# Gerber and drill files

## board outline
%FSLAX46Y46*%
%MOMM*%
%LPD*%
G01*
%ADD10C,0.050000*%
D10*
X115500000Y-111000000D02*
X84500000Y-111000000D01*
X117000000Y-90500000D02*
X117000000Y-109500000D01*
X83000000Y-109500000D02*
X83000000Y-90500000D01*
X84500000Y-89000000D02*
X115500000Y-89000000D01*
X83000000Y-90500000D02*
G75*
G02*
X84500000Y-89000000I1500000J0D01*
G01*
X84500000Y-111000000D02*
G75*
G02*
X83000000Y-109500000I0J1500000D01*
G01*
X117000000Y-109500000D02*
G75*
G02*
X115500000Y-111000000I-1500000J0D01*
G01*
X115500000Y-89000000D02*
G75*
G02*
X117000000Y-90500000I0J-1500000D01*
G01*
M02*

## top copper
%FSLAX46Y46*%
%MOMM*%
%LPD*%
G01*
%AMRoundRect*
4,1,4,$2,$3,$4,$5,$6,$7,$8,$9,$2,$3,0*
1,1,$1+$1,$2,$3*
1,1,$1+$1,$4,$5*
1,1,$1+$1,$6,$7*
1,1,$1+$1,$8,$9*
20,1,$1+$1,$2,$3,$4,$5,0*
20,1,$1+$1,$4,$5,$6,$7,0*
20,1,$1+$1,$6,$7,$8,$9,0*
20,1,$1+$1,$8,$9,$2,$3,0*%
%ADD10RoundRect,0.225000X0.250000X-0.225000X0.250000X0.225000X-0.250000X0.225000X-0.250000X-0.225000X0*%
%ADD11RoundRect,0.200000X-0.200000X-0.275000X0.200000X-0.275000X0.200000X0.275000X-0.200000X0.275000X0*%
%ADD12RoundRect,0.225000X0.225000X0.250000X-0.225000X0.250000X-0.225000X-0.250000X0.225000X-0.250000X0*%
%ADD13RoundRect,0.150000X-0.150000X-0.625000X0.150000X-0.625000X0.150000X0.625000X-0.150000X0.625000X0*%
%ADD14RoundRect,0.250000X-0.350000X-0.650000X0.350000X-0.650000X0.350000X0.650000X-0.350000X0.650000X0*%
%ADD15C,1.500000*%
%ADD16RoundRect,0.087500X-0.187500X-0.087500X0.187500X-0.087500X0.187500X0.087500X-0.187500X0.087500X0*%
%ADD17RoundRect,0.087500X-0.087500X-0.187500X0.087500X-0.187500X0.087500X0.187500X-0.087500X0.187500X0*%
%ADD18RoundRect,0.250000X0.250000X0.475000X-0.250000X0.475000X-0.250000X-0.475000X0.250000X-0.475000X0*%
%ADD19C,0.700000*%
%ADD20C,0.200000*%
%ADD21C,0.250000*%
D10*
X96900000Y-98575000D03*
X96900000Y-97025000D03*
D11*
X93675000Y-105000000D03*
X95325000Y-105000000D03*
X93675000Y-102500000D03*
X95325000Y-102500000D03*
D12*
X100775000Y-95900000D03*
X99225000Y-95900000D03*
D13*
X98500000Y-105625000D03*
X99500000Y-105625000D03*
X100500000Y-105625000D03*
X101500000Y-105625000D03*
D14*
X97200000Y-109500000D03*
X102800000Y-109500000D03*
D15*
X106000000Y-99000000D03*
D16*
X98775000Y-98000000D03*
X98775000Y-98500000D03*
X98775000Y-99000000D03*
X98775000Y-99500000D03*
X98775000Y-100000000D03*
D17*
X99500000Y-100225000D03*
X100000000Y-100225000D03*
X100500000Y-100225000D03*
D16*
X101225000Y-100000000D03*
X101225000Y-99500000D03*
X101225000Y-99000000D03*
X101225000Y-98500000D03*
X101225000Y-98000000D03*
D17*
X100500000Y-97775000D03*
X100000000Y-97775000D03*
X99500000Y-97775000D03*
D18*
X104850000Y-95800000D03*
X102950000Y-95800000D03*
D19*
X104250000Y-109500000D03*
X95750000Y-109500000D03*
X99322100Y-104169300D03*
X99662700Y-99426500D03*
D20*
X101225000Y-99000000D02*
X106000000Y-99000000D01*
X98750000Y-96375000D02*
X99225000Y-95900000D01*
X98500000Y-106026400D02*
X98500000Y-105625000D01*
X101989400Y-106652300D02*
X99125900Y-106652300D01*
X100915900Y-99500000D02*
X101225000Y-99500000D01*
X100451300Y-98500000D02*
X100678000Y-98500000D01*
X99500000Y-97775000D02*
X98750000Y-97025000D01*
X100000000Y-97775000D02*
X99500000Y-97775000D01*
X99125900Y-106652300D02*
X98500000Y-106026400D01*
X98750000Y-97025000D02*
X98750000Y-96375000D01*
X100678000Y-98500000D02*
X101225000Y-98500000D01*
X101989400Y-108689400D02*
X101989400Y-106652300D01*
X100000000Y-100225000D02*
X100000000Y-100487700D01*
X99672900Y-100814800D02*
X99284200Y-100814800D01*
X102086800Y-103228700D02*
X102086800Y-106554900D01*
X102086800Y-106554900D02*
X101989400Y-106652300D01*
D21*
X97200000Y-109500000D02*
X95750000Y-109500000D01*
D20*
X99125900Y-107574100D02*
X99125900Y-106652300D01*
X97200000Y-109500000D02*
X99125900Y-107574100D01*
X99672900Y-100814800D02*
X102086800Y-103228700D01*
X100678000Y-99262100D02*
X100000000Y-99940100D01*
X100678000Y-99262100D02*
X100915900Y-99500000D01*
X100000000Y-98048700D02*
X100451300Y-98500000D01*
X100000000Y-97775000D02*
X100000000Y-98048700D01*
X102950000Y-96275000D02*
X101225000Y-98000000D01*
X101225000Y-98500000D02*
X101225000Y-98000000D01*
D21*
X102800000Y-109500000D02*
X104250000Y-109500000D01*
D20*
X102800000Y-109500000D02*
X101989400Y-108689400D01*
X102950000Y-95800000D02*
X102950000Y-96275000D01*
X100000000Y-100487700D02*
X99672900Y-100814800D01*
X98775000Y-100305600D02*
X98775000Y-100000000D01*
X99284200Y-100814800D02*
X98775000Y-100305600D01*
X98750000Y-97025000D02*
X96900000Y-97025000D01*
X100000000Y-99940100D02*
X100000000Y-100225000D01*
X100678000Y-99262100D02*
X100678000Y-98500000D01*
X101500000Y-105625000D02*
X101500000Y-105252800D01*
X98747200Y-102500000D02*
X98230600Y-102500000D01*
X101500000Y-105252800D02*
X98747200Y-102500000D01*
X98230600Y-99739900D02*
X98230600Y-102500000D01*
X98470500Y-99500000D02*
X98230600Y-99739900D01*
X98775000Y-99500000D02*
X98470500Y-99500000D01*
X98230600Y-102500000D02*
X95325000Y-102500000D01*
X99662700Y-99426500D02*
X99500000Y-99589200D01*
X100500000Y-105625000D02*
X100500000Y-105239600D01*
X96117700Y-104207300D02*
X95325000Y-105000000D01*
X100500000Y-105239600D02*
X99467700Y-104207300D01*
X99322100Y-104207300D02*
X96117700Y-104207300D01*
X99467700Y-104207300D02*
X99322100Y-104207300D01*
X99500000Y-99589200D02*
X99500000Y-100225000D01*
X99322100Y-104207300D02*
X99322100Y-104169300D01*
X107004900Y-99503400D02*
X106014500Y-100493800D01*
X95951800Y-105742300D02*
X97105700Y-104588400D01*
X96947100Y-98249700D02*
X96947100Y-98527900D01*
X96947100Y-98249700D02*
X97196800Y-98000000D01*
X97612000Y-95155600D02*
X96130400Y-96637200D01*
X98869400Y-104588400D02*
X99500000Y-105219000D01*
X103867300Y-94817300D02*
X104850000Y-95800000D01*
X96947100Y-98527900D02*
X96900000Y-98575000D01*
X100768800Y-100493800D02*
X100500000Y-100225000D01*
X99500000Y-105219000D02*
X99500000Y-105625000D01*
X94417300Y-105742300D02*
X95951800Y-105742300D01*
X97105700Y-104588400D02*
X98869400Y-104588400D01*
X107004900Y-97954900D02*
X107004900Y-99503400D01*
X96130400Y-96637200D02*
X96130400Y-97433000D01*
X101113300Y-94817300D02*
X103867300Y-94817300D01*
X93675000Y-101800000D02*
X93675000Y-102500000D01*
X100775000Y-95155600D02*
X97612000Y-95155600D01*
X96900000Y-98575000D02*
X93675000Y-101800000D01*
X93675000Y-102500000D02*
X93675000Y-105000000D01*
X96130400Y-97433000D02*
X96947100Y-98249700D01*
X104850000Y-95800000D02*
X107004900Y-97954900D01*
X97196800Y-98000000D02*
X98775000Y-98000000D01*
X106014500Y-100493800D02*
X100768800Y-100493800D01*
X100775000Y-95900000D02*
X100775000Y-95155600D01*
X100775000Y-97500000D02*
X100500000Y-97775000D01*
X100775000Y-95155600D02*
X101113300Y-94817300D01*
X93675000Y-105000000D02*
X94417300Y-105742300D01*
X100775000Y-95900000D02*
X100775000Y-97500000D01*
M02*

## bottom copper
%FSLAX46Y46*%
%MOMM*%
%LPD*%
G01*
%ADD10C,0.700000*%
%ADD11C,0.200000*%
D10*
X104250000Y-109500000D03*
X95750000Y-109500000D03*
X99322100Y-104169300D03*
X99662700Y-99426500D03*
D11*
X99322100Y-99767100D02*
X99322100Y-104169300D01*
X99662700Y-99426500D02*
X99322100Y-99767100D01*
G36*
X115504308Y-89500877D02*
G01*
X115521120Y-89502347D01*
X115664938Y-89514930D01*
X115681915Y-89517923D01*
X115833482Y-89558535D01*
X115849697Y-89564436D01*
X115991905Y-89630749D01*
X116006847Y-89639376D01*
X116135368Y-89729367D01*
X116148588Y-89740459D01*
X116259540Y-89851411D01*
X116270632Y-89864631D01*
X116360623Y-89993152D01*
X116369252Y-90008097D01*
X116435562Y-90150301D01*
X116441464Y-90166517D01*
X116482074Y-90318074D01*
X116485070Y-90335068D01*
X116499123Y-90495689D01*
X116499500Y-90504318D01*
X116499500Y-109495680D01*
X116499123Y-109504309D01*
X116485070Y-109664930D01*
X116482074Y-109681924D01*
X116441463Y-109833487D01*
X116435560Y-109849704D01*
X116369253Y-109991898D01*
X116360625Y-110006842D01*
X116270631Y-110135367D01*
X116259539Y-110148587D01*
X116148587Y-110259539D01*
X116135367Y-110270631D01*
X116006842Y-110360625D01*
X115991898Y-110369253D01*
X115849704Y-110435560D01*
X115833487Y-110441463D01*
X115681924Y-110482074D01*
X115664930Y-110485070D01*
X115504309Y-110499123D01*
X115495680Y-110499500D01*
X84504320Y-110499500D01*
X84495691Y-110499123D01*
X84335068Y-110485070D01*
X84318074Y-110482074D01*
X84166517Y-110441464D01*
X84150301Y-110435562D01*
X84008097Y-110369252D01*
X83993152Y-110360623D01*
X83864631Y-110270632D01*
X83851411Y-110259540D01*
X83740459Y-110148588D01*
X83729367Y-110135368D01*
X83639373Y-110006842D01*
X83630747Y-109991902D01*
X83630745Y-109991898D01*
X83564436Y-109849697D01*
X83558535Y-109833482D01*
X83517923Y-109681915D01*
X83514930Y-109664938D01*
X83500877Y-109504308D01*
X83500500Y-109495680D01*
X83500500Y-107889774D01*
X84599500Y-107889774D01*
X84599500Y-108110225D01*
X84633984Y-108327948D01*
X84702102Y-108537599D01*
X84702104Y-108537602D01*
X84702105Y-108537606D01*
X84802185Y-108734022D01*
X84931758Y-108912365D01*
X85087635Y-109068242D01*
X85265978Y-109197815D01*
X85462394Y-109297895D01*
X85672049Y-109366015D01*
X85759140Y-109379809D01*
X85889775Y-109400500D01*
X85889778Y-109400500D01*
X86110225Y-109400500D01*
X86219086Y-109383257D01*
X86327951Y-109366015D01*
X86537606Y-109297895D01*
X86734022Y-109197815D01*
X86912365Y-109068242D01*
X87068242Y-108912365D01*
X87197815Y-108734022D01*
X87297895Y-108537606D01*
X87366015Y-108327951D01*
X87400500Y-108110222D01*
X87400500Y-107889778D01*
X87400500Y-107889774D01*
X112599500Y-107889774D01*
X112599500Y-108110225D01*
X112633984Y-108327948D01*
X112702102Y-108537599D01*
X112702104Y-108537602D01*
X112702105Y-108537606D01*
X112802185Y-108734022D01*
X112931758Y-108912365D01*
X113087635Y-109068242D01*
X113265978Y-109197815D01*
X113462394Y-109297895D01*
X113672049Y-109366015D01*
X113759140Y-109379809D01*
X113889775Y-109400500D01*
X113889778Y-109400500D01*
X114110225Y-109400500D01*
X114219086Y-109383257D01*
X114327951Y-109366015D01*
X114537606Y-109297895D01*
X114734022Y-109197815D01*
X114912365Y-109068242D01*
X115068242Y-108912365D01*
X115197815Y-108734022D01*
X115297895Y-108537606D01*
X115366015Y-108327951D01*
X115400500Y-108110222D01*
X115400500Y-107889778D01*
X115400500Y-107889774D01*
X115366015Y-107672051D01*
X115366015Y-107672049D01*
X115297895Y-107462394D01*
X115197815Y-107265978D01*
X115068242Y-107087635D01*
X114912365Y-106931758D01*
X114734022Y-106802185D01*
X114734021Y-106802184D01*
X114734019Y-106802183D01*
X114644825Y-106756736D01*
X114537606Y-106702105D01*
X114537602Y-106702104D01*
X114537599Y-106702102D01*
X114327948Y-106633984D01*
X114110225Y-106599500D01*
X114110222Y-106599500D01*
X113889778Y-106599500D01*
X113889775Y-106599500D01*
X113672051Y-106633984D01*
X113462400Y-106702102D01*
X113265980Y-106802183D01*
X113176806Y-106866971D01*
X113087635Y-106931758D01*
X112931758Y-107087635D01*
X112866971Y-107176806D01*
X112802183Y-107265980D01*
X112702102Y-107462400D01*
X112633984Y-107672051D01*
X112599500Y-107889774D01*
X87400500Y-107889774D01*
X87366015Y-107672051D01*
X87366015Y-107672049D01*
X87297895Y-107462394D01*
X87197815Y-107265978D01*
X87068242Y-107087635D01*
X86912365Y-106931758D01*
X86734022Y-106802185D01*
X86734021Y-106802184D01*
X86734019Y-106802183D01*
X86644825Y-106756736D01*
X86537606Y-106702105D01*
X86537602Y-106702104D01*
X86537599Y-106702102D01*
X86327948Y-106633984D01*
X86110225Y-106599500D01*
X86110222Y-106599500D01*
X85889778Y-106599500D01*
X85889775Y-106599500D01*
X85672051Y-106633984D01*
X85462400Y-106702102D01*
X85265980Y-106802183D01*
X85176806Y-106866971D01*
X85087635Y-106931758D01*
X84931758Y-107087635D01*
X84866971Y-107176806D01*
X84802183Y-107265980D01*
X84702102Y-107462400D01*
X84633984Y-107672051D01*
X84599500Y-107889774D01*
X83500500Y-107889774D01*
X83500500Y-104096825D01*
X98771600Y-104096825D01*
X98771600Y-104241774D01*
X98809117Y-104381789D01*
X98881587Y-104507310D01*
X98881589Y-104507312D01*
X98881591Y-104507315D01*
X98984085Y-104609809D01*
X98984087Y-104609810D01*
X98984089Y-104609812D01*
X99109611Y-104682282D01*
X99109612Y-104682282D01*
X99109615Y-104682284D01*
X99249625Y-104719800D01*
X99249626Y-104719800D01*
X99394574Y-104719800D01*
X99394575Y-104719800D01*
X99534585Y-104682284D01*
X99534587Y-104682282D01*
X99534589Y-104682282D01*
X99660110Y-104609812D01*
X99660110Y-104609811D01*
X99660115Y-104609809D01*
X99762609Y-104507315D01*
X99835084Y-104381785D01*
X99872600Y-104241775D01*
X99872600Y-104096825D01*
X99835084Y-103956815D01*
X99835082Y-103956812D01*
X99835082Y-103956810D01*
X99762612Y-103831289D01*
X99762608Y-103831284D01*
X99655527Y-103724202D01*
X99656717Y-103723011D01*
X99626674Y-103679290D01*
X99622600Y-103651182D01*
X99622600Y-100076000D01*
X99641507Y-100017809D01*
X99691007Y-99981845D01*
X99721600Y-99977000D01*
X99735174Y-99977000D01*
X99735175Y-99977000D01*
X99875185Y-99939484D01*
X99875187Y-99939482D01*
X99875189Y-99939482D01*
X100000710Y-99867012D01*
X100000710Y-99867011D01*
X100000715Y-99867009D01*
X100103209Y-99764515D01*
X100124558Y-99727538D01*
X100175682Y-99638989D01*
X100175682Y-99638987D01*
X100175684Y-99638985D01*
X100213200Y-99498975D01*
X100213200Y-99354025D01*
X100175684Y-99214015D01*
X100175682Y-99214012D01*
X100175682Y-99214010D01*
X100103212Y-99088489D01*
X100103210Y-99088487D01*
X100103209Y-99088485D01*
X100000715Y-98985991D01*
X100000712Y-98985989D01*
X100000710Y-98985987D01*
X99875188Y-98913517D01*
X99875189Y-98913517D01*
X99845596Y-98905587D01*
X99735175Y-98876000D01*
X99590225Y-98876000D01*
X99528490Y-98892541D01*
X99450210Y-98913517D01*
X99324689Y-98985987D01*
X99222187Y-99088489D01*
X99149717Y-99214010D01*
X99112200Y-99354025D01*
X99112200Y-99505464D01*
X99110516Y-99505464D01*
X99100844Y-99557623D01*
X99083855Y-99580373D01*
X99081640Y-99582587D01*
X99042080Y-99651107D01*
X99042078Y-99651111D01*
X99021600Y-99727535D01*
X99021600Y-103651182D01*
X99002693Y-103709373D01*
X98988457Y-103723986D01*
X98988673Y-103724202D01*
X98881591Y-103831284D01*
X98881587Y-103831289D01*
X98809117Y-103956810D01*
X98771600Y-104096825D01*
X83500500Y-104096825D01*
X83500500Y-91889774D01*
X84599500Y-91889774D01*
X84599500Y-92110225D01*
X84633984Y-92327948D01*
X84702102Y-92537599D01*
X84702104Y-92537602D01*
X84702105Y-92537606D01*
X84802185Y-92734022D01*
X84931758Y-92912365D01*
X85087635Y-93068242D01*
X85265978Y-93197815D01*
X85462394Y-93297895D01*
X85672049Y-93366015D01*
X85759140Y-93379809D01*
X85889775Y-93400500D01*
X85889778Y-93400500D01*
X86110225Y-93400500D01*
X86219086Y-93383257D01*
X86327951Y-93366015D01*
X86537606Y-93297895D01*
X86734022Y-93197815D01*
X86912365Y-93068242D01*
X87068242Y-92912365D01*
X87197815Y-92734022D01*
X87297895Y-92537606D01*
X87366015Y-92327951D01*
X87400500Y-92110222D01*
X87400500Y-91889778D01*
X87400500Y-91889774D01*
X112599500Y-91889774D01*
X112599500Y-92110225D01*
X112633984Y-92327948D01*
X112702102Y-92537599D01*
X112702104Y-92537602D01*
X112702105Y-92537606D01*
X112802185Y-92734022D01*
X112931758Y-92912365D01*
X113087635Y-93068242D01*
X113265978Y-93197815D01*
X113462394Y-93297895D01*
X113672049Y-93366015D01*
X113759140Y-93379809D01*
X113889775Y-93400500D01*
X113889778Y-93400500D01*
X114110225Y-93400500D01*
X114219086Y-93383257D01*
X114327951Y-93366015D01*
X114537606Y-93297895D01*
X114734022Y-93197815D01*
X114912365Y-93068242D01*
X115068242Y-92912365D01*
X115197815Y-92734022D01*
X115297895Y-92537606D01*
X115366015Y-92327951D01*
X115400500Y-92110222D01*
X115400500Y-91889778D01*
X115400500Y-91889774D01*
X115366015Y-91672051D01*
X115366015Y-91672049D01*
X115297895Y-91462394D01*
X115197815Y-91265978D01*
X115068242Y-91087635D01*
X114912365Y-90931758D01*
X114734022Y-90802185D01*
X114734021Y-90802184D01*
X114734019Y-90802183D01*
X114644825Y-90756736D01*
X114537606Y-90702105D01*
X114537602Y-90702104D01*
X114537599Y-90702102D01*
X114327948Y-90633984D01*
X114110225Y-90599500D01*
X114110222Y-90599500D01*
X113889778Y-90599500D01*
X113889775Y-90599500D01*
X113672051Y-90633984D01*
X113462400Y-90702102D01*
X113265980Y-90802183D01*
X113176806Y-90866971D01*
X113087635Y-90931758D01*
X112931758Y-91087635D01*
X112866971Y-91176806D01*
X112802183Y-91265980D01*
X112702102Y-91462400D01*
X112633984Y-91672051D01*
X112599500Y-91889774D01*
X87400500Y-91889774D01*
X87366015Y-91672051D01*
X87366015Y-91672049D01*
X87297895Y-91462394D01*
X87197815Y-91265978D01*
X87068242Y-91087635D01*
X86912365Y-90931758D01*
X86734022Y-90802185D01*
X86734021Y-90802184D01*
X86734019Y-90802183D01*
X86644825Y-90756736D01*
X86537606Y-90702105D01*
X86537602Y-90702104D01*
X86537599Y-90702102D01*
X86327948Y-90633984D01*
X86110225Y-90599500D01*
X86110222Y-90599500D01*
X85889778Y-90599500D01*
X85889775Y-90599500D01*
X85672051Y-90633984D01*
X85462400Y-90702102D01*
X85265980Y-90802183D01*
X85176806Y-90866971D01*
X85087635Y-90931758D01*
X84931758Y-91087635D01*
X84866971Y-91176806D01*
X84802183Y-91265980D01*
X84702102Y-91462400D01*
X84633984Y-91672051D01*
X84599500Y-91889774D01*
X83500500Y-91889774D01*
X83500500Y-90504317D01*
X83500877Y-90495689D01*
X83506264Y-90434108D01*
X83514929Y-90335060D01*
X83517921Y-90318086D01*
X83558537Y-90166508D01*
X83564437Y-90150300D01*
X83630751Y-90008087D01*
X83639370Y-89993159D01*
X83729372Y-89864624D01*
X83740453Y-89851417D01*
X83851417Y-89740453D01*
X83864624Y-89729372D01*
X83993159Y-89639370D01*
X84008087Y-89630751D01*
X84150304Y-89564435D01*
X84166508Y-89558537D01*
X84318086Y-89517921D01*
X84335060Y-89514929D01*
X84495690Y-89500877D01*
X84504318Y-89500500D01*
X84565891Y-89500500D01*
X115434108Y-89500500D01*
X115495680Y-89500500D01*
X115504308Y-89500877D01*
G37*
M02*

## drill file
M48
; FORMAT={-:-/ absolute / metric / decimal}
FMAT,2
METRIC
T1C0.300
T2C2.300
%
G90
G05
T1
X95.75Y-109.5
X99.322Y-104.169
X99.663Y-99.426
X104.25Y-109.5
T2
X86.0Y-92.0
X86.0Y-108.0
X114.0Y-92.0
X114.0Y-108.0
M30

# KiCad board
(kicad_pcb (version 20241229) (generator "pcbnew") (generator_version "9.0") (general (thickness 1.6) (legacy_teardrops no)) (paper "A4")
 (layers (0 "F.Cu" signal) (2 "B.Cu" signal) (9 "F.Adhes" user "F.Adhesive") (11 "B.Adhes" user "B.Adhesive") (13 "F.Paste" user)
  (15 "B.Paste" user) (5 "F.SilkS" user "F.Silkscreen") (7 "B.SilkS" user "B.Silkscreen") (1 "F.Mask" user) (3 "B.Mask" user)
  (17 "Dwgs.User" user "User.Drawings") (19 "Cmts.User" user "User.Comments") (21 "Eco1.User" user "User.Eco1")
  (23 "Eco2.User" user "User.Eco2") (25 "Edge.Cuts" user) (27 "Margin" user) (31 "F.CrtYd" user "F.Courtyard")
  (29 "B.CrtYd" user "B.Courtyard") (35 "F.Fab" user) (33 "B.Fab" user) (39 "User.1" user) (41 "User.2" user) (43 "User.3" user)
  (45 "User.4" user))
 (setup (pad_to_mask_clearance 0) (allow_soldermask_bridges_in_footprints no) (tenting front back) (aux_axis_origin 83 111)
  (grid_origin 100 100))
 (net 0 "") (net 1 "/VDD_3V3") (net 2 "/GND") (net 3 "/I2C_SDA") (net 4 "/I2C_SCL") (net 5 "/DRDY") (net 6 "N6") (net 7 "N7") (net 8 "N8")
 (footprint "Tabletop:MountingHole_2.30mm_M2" (layer "F.Cu") (at 86 108)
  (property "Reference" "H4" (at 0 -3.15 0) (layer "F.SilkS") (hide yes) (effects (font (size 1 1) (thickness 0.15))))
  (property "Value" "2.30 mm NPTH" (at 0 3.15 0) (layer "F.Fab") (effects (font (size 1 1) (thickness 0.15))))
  (pad "" np_thru_hole circle (at 0 0) (size 2.3 2.3) (drill 2.3) (layers "*.Cu" "*.Mask")))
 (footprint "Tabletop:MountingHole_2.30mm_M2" (layer "F.Cu") (at 114 92)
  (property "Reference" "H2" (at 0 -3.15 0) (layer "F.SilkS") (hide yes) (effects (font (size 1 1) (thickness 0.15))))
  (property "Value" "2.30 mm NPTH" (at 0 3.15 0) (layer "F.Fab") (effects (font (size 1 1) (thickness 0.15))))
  (pad "" np_thru_hole circle (at 0 0) (size 2.3 2.3) (drill 2.3) (layers "*.Cu" "*.Mask")))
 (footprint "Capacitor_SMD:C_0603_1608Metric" (layer "F.Cu") (at 96.9 97.8 90)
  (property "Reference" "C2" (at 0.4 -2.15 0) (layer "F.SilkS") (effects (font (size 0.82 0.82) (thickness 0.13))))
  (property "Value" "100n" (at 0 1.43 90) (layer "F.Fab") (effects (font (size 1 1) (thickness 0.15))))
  (pad "1" smd roundrect (at -0.775 0 90) (size 0.9 0.95) (layers "F.Cu" "F.Mask" "F.Paste") (roundrect_rratio 0.25) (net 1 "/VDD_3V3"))
  (pad "2" smd roundrect (at 0.775 0 90) (size 0.9 0.95) (layers "F.Cu" "F.Mask" "F.Paste") (roundrect_rratio 0.25) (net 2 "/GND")))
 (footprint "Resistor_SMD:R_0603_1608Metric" (layer "F.Cu") (at 94.5 105)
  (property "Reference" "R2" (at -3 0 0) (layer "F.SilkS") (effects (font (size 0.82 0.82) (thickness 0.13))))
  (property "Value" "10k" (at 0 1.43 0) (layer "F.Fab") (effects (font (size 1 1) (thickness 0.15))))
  (pad "1" smd roundrect (at -0.825 0) (size 0.8 0.95) (layers "F.Cu" "F.Mask" "F.Paste") (roundrect_rratio 0.25) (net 1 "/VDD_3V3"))
  (pad "2" smd roundrect (at 0.825 0) (size 0.8 0.95) (layers "F.Cu" "F.Mask" "F.Paste") (roundrect_rratio 0.25) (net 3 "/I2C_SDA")))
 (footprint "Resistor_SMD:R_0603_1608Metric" (layer "F.Cu") (at 94.5 102.5)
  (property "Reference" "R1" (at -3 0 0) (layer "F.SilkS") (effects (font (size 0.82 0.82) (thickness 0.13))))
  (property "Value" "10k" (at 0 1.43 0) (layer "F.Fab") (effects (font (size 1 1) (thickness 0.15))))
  (pad "1" smd roundrect (at -0.825 0) (size 0.8 0.95) (layers "F.Cu" "F.Mask" "F.Paste") (roundrect_rratio 0.25) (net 1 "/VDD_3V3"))
  (pad "2" smd roundrect (at 0.825 0) (size 0.8 0.95) (layers "F.Cu" "F.Mask" "F.Paste") (roundrect_rratio 0.25) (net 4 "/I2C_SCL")))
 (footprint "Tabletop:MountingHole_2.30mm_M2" (layer "F.Cu") (at 114 108)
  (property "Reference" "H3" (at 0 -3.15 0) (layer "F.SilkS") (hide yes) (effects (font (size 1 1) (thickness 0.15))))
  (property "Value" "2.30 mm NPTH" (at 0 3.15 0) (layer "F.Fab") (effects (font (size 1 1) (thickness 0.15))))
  (pad "" np_thru_hole circle (at 0 0) (size 2.3 2.3) (drill 2.3) (layers "*.Cu" "*.Mask")))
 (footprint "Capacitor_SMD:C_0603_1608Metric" (layer "F.Cu") (at 100 95.9 180)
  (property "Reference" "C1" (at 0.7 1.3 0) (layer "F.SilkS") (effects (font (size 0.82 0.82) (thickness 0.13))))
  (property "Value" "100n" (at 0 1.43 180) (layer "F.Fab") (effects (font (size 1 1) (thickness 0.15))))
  (pad "1" smd roundrect (at -0.775 0 180) (size 0.9 0.95) (layers "F.Cu" "F.Mask" "F.Paste") (roundrect_rratio 0.25) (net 1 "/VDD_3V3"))
  (pad "2" smd roundrect (at 0.775 0 180) (size 0.9 0.95) (layers "F.Cu" "F.Mask" "F.Paste") (roundrect_rratio 0.25) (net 2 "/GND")))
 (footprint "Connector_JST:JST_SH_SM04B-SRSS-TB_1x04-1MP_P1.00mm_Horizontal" (layer "F.Cu") (at 100 107.625)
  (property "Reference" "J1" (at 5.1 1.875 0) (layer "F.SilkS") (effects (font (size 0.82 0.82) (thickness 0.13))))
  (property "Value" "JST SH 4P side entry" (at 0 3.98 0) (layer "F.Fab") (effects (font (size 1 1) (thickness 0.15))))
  (pad "1" smd roundrect (at -1.5 -2) (size 0.6 1.55) (layers "F.Cu" "F.Mask" "F.Paste") (roundrect_rratio 0.25) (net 2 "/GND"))
  (pad "2" smd roundrect (at -0.5 -2) (size 0.6 1.55) (layers "F.Cu" "F.Mask" "F.Paste") (roundrect_rratio 0.25) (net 1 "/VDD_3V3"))
  (pad "3" smd roundrect (at 0.5 -2) (size 0.6 1.55) (layers "F.Cu" "F.Mask" "F.Paste") (roundrect_rratio 0.25) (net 3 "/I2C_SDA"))
  (pad "4" smd roundrect (at 1.5 -2) (size 0.6 1.55) (layers "F.Cu" "F.Mask" "F.Paste") (roundrect_rratio 0.25) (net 4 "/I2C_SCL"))
  (pad "MP" smd roundrect (at -2.8 1.875) (size 1.2 1.8) (layers "F.Cu" "F.Mask" "F.Paste") (roundrect_rratio 0.208333) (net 2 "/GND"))
  (pad "MP" smd roundrect (at 2.8 1.875) (size 1.2 1.8) (layers "F.Cu" "F.Mask" "F.Paste") (roundrect_rratio 0.208333) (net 2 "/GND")))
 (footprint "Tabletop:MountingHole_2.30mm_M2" (layer "F.Cu") (at 86 92)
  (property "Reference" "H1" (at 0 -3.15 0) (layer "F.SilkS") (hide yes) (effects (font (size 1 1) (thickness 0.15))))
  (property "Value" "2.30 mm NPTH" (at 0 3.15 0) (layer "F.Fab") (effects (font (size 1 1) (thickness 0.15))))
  (pad "" np_thru_hole circle (at 0 0) (size 2.3 2.3) (drill 2.3) (layers "*.Cu" "*.Mask")))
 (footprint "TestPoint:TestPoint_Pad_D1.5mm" (layer "F.Cu") (at 106 99)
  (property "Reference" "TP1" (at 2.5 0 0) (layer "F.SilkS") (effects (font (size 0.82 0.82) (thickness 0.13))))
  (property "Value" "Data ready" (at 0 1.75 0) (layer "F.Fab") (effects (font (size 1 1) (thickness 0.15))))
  (pad "1" smd circle (at 0 0) (size 1.5 1.5) (layers "F.Cu" "F.Mask") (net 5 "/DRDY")))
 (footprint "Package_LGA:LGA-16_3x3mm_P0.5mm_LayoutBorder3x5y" (layer "F.Cu") (at 100 99)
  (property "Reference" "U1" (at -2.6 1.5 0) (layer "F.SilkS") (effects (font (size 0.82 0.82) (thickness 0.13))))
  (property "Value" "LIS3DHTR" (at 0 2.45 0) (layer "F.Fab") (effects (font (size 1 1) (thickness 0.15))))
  (pad "1" smd roundrect (at -1.225 -1) (size 0.55 0.35) (layers "F.Cu" "F.Mask" "F.Paste") (roundrect_rratio 0.25) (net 1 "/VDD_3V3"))
  (pad "2" smd roundrect (at -1.225 -0.5) (size 0.55 0.35) (layers "F.Cu" "F.Mask" "F.Paste") (roundrect_rratio 0.25) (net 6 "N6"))
  (pad "3" smd roundrect (at -1.225 0) (size 0.55 0.35) (layers "F.Cu" "F.Mask" "F.Paste") (roundrect_rratio 0.25) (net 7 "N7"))
  (pad "4" smd roundrect (at -1.225 0.5) (size 0.55 0.35) (layers "F.Cu" "F.Mask" "F.Paste") (roundrect_rratio 0.25) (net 4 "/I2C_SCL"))
  (pad "5" smd roundrect (at -1.225 1) (size 0.55 0.35) (layers "F.Cu" "F.Mask" "F.Paste") (roundrect_rratio 0.25) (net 2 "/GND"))
  (pad "6" smd roundrect (at -0.5 1.225) (size 0.35 0.55) (layers "F.Cu" "F.Mask" "F.Paste") (roundrect_rratio 0.25) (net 3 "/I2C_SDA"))
  (pad "7" smd roundrect (at 0 1.225) (size 0.35 0.55) (layers "F.Cu" "F.Mask" "F.Paste") (roundrect_rratio 0.25) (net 2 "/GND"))
  (pad "8" smd roundrect (at 0.5 1.225) (size 0.35 0.55) (layers "F.Cu" "F.Mask" "F.Paste") (roundrect_rratio 0.25) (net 1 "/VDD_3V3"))
  (pad "9" smd roundrect (at 1.225 1) (size 0.55 0.35) (layers "F.Cu" "F.Mask" "F.Paste") (roundrect_rratio 0.25) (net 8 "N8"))
  (pad "10" smd roundrect (at 1.225 0.5) (size 0.55 0.35) (layers "F.Cu" "F.Mask" "F.Paste") (roundrect_rratio 0.25) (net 2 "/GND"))
  (pad "11" smd roundrect (at 1.225 0) (size 0.55 0.35) (layers "F.Cu" "F.Mask" "F.Paste") (roundrect_rratio 0.25) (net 5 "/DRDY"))
  (pad "12" smd roundrect (at 1.225 -0.5) (size 0.55 0.35) (layers "F.Cu" "F.Mask" "F.Paste") (roundrect_rratio 0.25) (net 2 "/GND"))
  (pad "13" smd roundrect (at 1.225 -1) (size 0.55 0.35) (layers "F.Cu" "F.Mask" "F.Paste") (roundrect_rratio 0.25) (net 2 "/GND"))
  (pad "14" smd roundrect (at 0.5 -1.225) (size 0.35 0.55) (layers "F.Cu" "F.Mask" "F.Paste") (roundrect_rratio 0.25) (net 1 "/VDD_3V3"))
  (pad "15" smd roundrect (at 0 -1.225) (size 0.35 0.55) (layers "F.Cu" "F.Mask" "F.Paste") (roundrect_rratio 0.25) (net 2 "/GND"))
  (pad "16" smd roundrect (at -0.5 -1.225) (size 0.35 0.55) (layers "F.Cu" "F.Mask" "F.Paste") (roundrect_rratio 0.25) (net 2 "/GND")))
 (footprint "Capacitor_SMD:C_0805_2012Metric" (layer "F.Cu") (at 103.9 95.8 180)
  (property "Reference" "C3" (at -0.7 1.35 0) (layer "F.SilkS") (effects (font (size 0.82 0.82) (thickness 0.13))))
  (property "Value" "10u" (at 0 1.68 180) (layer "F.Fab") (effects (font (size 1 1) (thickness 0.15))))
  (pad "1" smd roundrect (at -0.95 0 180) (size 1 1.45) (layers "F.Cu" "F.Mask" "F.Paste") (roundrect_rratio 0.25) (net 1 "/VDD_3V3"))
  (pad "2" smd roundrect (at 0.95 0 180) (size 1 1.45) (layers "F.Cu" "F.Mask" "F.Paste") (roundrect_rratio 0.25) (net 2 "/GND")))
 (gr_line (start 115.5 111) (end 84.5 111) (stroke (width 0.05) (type default)) (layer "Edge.Cuts"))
 (gr_line (start 117 90.5) (end 117 109.5) (stroke (width 0.05) (type default)) (layer "Edge.Cuts"))
 (gr_line (start 83 109.5) (end 83 90.5) (stroke (width 0.05) (type default)) (layer "Edge.Cuts"))
 (gr_line (start 84.5 89) (end 115.5 89) (stroke (width 0.05) (type default)) (layer "Edge.Cuts"))
 (gr_arc (start 83 90.5) (mid 83.439339 89.439339) (end 84.5 89) (stroke (width 0.05) (type default)) (layer "Edge.Cuts"))
 (gr_arc (start 84.5 111) (mid 83.439339 110.56066) (end 83 109.5) (stroke (width 0.05) (type default)) (layer "Edge.Cuts"))
 (gr_arc (start 117 109.5) (mid 116.56066 110.56066) (end 115.5 111) (stroke (width 0.05) (type default)) (layer "Edge.Cuts"))
 (gr_arc (start 115.5 89) (mid 116.56066 89.439339) (end 117 90.5) (stroke (width 0.05) (type default)) (layer "Edge.Cuts"))
 (segment (start 101.225 99) (end 106 99) (width 0.2) (layer "F.Cu") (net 5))
 (segment (start 98.75 96.375) (end 99.225 95.9) (width 0.2) (layer "F.Cu") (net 2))
 (segment (start 98.5 106.0264) (end 98.5 105.625) (width 0.2) (layer "F.Cu") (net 2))
 (segment (start 101.9894 106.6523) (end 99.1259 106.6523) (width 0.2) (layer "F.Cu") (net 2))
 (segment (start 100.9159 99.5) (end 101.225 99.5) (width 0.2) (layer "F.Cu") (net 2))
 (segment (start 100.4513 98.5) (end 100.678 98.5) (width 0.2) (layer "F.Cu") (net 2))
 (segment (start 99.5 97.775) (end 98.75 97.025) (width 0.2) (layer "F.Cu") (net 2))
 (segment (start 100 97.775) (end 99.5 97.775) (width 0.2) (layer "F.Cu") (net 2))
 (segment (start 99.1259 106.6523) (end 98.5 106.0264) (width 0.2) (layer "F.Cu") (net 2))
 (segment (start 98.75 97.025) (end 98.75 96.375) (width 0.2) (layer "F.Cu") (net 2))
 (segment (start 100.678 98.5) (end 101.225 98.5) (width 0.2) (layer "F.Cu") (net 2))
 (segment (start 101.9894 108.6894) (end 101.9894 106.6523) (width 0.2) (layer "F.Cu") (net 2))
 (segment (start 100 100.225) (end 100 100.4877) (width 0.2) (layer "F.Cu") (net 2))
 (segment (start 99.6729 100.8148) (end 99.2842 100.8148) (width 0.2) (layer "F.Cu") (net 2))
 (segment (start 102.0868 103.2287) (end 102.0868 106.5549) (width 0.2) (layer "F.Cu") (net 2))
 (segment (start 102.0868 106.5549) (end 101.9894 106.6523) (width 0.2) (layer "F.Cu") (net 2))
 (segment (start 97.2 109.5) (end 95.75 109.5) (width 0.25) (layer "F.Cu") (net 2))
 (segment (start 99.1259 107.5741) (end 99.1259 106.6523) (width 0.2) (layer "F.Cu") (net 2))
 (segment (start 97.2 109.5) (end 99.1259 107.5741) (width 0.2) (layer "F.Cu") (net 2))
 (segment (start 99.6729 100.8148) (end 102.0868 103.2287) (width 0.2) (layer "F.Cu") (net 2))
 (segment (start 100.678 99.2621) (end 100 99.9401) (width 0.2) (layer "F.Cu") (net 2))
 (segment (start 100.678 99.2621) (end 100.9159 99.5) (width 0.2) (layer "F.Cu") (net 2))
 (segment (start 100 98.0487) (end 100.4513 98.5) (width 0.2) (layer "F.Cu") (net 2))
 (segment (start 100 97.775) (end 100 98.0487) (width 0.2) (layer "F.Cu") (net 2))
 (segment (start 102.95 96.275) (end 101.225 98) (width 0.2) (layer "F.Cu") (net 2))
 (segment (start 101.225 98.5) (end 101.225 98) (width 0.2) (layer "F.Cu") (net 2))
 (segment (start 102.8 109.5) (end 104.25 109.5) (width 0.25) (layer "F.Cu") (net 2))
 (segment (start 102.8 109.5) (end 101.9894 108.6894) (width 0.2) (layer "F.Cu") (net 2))
 (segment (start 102.95 95.8) (end 102.95 96.275) (width 0.2) (layer "F.Cu") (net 2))
 (segment (start 100 100.4877) (end 99.6729 100.8148) (width 0.2) (layer "F.Cu") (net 2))
 (segment (start 98.775 100.3056) (end 98.775 100) (width 0.2) (layer "F.Cu") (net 2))
 (segment (start 99.2842 100.8148) (end 98.775 100.3056) (width 0.2) (layer "F.Cu") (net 2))
 (segment (start 98.75 97.025) (end 96.9 97.025) (width 0.2) (layer "F.Cu") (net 2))
 (segment (start 100 99.9401) (end 100 100.225) (width 0.2) (layer "F.Cu") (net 2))
 (segment (start 100.678 99.2621) (end 100.678 98.5) (width 0.2) (layer "F.Cu") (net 2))
 (via (at 104.25 109.5) (size 0.7) (drill 0.3) (layers "F.Cu" "B.Cu") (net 2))
 (via (at 95.75 109.5) (size 0.7) (drill 0.3) (layers "F.Cu" "B.Cu") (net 2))
 (segment (start 101.5 105.625) (end 101.5 105.2528) (width 0.2) (layer "F.Cu") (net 4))
 (segment (start 98.7472 102.5) (end 98.2306 102.5) (width 0.2) (layer "F.Cu") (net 4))
 (segment (start 101.5 105.2528) (end 98.7472 102.5) (width 0.2) (layer "F.Cu") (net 4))
 (segment (start 98.2306 99.7399) (end 98.2306 102.5) (width 0.2) (layer "F.Cu") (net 4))
 (segment (start 98.4705 99.5) (end 98.2306 99.7399) (width 0.2) (layer "F.Cu") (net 4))
 (segment (start 98.775 99.5) (end 98.4705 99.5) (width 0.2) (layer "F.Cu") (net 4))
 (segment (start 98.2306 102.5) (end 95.325 102.5) (width 0.2) (layer "F.Cu") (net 4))
 (segment (start 99.6627 99.4265) (end 99.5 99.5892) (width 0.2) (layer "F.Cu") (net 3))
 (segment (start 100.5 105.625) (end 100.5 105.2396) (width 0.2) (layer "F.Cu") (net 3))
 (segment (start 96.1177 104.2073) (end 95.325 105) (width 0.2) (layer "F.Cu") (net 3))
 (segment (start 100.5 105.2396) (end 99.4677 104.2073) (width 0.2) (layer "F.Cu") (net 3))
 (segment (start 99.3221 104.2073) (end 96.1177 104.2073) (width 0.2) (layer "F.Cu") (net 3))
 (segment (start 99.4677 104.2073) (end 99.3221 104.2073) (width 0.2) (layer "F.Cu") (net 3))
 (segment (start 99.5 99.5892) (end 99.5 100.225) (width 0.2) (layer "F.Cu") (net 3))
 (segment (start 99.3221 104.2073) (end 99.3221 104.1693) (width 0.2) (layer "F.Cu") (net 3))
 (via (at 99.3221 104.1693) (size 0.7) (drill 0.3) (layers "F.Cu" "B.Cu") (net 3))
 (via (at 99.6627 99.4265) (size 0.7) (drill 0.3) (layers "F.Cu" "B.Cu") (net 3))
 (segment (start 99.3221 99.7671) (end 99.3221 104.1693) (width 0.2) (layer "B.Cu") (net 3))
 (segment (start 99.6627 99.4265) (end 99.3221 99.7671) (width 0.2) (layer "B.Cu") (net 3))
 (segment (start 107.0049 99.5034) (end 106.0145 100.4938) (width 0.2) (layer "F.Cu") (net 1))
 (segment (start 95.9518 105.7423) (end 97.1057 104.5884) (width 0.2) (layer "F.Cu") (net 1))
 (segment (start 96.9471 98.2497) (end 96.9471 98.5279) (width 0.2) (layer "F.Cu") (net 1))
 (segment (start 96.9471 98.2497) (end 97.1968 98) (width 0.2) (layer "F.Cu") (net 1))
 (segment (start 97.612 95.1556) (end 96.1304 96.6372) (width 0.2) (layer "F.Cu") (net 1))
 (segment (start 98.8694 104.5884) (end 99.5 105.219) (width 0.2) (layer "F.Cu") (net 1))
 (segment (start 103.8673 94.8173) (end 104.85 95.8) (width 0.2) (layer "F.Cu") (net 1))
 (segment (start 96.9471 98.5279) (end 96.9 98.575) (width 0.2) (layer "F.Cu") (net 1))
 (segment (start 100.7688 100.4938) (end 100.5 100.225) (width 0.2) (layer "F.Cu") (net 1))
 (segment (start 99.5 105.219) (end 99.5 105.625) (width 0.2) (layer "F.Cu") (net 1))
 (segment (start 94.4173 105.7423) (end 95.9518 105.7423) (width 0.2) (layer "F.Cu") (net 1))
 (segment (start 97.1057 104.5884) (end 98.8694 104.5884) (width 0.2) (layer "F.Cu") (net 1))
 (segment (start 107.0049 97.9549) (end 107.0049 99.5034) (width 0.2) (layer "F.Cu") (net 1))
 (segment (start 96.1304 96.6372) (end 96.1304 97.433) (width 0.2) (layer "F.Cu") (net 1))
 (segment (start 101.1133 94.8173) (end 103.8673 94.8173) (width 0.2) (layer "F.Cu") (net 1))
 (segment (start 93.675 101.8) (end 93.675 102.5) (width 0.2) (layer "F.Cu") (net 1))
 (segment (start 100.775 95.1556) (end 97.612 95.1556) (width 0.2) (layer "F.Cu") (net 1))
 (segment (start 96.9 98.575) (end 93.675 101.8) (width 0.2) (layer "F.Cu") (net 1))
 (segment (start 93.675 102.5) (end 93.675 105) (width 0.2) (layer "F.Cu") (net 1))
 (segment (start 96.1304 97.433) (end 96.9471 98.2497) (width 0.2) (layer "F.Cu") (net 1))
 (segment (start 104.85 95.8) (end 107.0049 97.9549) (width 0.2) (layer "F.Cu") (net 1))
 (segment (start 97.1968 98) (end 98.775 98) (width 0.2) (layer "F.Cu") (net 1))
 (segment (start 106.0145 100.4938) (end 100.7688 100.4938) (width 0.2) (layer "F.Cu") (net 1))
 (segment (start 100.775 95.9) (end 100.775 95.1556) (width 0.2) (layer "F.Cu") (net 1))
 (segment (start 100.775 97.5) (end 100.5 97.775) (width 0.2) (layer "F.Cu") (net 1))
 (segment (start 100.775 95.1556) (end 101.1133 94.8173) (width 0.2) (layer "F.Cu") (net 1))
 (segment (start 93.675 105) (end 94.4173 105.7423) (width 0.2) (layer "F.Cu") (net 1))
 (segment (start 100.775 95.9) (end 100.775 97.5) (width 0.2) (layer "F.Cu") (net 1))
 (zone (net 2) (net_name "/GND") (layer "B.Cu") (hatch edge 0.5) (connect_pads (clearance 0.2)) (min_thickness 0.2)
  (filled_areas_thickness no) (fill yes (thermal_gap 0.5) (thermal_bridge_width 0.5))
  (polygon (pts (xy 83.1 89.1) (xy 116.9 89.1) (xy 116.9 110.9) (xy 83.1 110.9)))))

